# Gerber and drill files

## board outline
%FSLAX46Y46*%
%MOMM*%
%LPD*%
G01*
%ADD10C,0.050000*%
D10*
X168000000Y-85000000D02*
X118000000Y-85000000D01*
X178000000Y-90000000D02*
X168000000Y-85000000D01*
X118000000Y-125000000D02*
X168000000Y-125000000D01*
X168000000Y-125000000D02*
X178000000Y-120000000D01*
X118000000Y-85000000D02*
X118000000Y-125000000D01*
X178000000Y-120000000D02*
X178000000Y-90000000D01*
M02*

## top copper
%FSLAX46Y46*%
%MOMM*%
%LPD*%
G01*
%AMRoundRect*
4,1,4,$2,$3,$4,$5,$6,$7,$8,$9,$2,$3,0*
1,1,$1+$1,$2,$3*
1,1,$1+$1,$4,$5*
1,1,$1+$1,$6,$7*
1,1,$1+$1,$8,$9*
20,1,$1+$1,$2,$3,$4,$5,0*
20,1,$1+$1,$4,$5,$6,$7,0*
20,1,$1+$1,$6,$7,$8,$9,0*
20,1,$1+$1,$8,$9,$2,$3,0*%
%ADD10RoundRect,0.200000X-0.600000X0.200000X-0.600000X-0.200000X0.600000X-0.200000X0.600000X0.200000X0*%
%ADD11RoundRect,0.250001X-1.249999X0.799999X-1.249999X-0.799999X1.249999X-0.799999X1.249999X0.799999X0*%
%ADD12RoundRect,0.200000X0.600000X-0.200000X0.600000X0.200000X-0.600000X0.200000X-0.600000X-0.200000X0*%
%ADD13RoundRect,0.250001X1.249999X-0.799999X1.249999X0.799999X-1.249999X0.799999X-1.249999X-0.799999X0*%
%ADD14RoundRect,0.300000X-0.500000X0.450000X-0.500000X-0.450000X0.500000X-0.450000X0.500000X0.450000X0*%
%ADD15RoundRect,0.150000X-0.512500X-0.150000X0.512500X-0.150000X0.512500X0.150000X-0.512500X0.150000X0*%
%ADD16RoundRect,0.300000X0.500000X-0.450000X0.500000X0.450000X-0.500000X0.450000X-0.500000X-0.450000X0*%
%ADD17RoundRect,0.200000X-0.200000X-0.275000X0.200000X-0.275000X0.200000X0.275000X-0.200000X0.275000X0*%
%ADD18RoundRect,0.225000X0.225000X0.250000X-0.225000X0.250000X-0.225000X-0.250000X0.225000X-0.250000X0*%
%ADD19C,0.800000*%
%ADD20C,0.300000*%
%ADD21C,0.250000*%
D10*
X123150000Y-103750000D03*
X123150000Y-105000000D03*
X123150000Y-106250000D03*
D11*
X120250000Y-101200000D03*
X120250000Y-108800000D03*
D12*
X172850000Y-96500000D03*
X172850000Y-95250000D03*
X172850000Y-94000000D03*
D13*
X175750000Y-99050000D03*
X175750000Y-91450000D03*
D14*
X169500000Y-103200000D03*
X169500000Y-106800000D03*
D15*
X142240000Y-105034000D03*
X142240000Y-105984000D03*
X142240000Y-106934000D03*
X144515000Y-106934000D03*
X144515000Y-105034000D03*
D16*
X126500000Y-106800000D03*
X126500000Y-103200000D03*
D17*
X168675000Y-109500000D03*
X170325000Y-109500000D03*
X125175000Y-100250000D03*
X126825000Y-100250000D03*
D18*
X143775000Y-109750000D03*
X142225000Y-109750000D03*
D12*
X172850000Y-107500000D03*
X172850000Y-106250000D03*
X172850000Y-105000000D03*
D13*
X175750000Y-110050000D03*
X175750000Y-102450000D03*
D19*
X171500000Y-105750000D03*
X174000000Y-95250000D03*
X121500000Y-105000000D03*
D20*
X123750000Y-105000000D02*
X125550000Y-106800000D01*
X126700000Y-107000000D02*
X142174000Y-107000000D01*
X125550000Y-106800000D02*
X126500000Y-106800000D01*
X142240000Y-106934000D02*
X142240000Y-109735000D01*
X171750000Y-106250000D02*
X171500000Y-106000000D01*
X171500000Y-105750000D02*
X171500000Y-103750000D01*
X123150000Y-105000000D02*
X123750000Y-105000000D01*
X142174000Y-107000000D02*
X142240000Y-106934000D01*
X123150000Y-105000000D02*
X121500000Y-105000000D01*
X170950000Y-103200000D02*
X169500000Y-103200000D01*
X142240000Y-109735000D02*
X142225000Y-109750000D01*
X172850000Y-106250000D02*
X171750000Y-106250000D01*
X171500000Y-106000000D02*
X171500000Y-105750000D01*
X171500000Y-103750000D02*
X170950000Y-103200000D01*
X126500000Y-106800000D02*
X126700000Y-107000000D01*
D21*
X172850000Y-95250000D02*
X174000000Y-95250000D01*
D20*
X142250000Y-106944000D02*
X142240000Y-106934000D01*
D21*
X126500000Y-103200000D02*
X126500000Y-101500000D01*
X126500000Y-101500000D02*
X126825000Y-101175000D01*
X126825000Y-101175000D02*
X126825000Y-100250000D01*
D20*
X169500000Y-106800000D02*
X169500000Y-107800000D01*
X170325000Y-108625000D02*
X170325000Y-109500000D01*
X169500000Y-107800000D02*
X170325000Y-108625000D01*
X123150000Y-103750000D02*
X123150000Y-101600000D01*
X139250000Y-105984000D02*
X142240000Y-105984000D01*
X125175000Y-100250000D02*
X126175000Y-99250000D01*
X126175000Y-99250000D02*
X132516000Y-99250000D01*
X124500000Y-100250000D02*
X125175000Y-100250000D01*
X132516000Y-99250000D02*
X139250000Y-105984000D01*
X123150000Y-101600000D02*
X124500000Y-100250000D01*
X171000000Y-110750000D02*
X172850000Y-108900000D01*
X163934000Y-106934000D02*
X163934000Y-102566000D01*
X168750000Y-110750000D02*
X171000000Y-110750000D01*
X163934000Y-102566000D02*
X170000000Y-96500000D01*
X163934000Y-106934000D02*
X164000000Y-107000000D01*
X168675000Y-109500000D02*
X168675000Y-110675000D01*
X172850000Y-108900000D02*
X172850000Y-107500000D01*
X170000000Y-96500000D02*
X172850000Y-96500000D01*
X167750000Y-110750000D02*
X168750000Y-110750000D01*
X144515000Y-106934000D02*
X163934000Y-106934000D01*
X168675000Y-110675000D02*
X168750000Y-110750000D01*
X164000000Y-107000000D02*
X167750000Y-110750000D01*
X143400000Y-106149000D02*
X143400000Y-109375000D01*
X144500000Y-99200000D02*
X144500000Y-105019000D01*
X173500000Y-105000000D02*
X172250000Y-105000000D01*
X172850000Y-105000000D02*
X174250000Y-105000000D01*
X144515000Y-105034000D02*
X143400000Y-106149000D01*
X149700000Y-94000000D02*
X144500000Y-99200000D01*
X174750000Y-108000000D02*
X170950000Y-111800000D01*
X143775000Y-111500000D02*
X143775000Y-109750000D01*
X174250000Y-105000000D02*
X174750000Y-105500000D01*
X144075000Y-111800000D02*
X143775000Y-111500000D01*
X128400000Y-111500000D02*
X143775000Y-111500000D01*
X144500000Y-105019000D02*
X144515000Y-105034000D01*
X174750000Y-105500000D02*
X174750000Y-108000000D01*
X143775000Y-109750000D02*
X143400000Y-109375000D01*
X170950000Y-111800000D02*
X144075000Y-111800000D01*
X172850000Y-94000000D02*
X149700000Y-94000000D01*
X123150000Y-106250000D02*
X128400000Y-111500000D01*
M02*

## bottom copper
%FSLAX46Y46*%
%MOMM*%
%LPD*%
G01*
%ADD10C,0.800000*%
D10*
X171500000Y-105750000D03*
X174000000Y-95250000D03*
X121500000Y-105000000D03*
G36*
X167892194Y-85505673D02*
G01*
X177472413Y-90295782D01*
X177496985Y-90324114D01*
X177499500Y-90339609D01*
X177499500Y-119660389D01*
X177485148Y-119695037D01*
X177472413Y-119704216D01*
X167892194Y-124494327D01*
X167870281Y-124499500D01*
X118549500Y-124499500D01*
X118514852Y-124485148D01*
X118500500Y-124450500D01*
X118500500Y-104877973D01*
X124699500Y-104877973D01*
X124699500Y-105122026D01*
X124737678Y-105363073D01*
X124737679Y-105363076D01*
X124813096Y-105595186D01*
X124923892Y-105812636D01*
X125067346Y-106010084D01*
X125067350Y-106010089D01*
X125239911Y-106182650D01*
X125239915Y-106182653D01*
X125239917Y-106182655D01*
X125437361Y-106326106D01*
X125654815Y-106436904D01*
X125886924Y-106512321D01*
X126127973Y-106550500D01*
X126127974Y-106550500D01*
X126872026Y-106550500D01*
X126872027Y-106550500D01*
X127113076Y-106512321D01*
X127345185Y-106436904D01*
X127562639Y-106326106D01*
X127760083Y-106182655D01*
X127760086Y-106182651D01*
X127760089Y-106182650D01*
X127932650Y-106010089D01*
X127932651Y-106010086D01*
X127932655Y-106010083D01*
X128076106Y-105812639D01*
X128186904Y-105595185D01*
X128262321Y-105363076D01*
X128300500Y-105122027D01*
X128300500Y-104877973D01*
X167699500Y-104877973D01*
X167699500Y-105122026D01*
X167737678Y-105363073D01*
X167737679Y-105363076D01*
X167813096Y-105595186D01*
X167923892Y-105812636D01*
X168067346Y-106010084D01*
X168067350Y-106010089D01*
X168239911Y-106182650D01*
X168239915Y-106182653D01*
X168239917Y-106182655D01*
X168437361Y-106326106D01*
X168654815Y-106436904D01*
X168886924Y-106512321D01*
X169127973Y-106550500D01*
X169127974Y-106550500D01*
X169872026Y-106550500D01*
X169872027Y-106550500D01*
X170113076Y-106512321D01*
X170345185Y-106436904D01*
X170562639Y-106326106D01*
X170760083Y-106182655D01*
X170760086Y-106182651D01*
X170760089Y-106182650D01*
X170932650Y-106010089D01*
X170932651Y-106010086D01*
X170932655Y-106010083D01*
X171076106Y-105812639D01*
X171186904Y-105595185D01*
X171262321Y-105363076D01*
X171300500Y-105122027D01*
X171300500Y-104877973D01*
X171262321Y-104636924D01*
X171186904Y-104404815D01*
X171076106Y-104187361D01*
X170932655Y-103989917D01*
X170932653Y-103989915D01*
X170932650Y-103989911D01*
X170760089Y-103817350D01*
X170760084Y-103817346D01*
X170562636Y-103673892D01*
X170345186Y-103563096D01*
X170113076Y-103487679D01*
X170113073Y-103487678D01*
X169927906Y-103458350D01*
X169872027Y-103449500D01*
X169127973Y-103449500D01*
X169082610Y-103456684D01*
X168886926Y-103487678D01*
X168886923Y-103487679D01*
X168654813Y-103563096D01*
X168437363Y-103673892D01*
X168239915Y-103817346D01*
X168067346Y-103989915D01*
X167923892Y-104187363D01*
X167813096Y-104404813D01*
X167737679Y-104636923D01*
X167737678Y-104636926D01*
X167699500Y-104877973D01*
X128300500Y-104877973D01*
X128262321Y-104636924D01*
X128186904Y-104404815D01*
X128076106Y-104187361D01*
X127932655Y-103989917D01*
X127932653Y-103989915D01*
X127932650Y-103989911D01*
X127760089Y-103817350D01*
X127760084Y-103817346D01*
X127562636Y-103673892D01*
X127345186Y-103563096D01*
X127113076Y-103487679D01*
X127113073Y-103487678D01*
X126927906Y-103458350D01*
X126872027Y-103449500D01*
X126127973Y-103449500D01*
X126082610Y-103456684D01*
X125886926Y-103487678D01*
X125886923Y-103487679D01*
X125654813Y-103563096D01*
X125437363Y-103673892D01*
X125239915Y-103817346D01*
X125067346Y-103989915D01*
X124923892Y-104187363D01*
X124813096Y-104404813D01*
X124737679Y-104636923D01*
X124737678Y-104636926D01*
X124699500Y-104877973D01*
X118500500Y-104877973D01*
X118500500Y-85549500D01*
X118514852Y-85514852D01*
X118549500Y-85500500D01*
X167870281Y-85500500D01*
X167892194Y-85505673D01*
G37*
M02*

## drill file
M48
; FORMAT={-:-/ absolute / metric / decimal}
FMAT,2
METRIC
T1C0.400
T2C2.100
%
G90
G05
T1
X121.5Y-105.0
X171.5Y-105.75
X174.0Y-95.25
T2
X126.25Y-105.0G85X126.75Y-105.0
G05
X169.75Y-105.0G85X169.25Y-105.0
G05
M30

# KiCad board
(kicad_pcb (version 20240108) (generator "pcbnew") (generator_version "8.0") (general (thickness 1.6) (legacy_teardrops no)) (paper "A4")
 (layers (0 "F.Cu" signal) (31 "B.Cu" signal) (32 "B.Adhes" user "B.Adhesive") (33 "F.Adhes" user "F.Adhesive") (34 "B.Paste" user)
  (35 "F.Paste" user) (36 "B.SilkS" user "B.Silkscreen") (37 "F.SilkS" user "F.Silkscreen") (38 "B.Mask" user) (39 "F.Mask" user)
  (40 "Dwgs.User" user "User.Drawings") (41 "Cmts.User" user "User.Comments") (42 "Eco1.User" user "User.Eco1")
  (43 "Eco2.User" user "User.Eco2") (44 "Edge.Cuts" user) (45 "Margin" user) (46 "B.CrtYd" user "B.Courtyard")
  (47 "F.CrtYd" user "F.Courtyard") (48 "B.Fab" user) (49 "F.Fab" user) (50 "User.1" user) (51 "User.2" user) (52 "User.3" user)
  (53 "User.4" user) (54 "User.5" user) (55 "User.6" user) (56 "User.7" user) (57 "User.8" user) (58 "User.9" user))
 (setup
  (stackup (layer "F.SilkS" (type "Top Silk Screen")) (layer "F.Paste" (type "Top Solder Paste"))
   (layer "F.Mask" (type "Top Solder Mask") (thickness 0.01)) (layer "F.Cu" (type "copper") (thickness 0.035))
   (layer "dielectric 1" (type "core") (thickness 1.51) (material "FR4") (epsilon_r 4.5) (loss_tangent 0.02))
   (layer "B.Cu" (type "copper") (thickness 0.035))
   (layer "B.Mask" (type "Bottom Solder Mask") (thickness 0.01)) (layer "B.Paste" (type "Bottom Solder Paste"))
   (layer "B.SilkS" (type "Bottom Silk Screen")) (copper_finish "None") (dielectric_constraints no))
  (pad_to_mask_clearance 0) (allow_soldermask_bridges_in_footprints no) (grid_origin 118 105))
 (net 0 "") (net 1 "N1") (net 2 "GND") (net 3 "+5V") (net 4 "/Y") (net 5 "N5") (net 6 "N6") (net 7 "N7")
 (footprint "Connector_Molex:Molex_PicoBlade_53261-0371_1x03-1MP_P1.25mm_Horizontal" (layer "F.Cu") (at 120.75 105 -90)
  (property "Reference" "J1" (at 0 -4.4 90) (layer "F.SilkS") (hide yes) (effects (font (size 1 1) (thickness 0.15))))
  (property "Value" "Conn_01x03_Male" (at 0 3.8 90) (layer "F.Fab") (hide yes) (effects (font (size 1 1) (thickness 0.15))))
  (pad "1" smd roundrect (at -1.25 -2.4 270) (size 0.8 1.6) (layers "F.Cu" "F.Paste" "F.Mask") (roundrect_rratio 0.25) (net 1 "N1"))
  (pad "2" smd roundrect (at 0 -2.4 270) (size 0.8 1.6) (layers "F.Cu" "F.Paste" "F.Mask") (roundrect_rratio 0.25) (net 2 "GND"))
  (pad "3" smd roundrect (at 1.25 -2.4 270) (size 0.8 1.6) (layers "F.Cu" "F.Paste" "F.Mask") (roundrect_rratio 0.25) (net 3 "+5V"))
  (pad "MP" smd roundrect (at -3.8 0.5 270) (size 2.1 3) (layers "F.Cu" "F.Paste" "F.Mask") (roundrect_rratio 0.1190480952))
  (pad "MP" smd roundrect (at 3.8 0.5 270) (size 2.1 3) (layers "F.Cu" "F.Paste" "F.Mask") (roundrect_rratio 0.1190480952)))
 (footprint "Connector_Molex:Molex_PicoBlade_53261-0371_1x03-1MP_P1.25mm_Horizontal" (layer "F.Cu") (at 175.25 95.25 90)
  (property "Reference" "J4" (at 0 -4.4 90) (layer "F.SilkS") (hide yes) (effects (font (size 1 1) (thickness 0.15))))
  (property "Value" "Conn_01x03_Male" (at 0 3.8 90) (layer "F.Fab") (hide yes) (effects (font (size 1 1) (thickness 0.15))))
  (pad "1" smd roundrect (at -1.25 -2.4 90) (size 0.8 1.6) (layers "F.Cu" "F.Paste" "F.Mask") (roundrect_rratio 0.25) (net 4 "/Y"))
  (pad "2" smd roundrect (at 0 -2.4 90) (size 0.8 1.6) (layers "F.Cu" "F.Paste" "F.Mask") (roundrect_rratio 0.25) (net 2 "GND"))
  (pad "3" smd roundrect (at 1.25 -2.4 90) (size 0.8 1.6) (layers "F.Cu" "F.Paste" "F.Mask") (roundrect_rratio 0.25) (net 3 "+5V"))
  (pad "MP" smd roundrect (at -3.8 0.5 90) (size 2.1 3) (layers "F.Cu" "F.Paste" "F.Mask") (roundrect_rratio 0.1190480952))
  (pad "MP" smd roundrect (at 3.8 0.5 90) (size 2.1 3) (layers "F.Cu" "F.Paste" "F.Mask") (roundrect_rratio 0.1190480952)))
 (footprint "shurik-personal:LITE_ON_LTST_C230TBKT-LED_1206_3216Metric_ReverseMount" (layer "F.Cu") (at 169.5 105 -90)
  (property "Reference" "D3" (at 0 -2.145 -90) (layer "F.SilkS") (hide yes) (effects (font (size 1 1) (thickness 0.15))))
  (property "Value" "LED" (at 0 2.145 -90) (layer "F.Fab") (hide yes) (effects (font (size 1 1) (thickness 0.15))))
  (pad "" np_thru_hole oval (at 0 0 270) (size 2.1 2.6) (drill oval 2.1 2.6) (layers "F&B.Cu" "*.Mask"))
  (pad "1" smd roundrect (at -1.8 0 270) (size 1.5 1.6) (layers "F.Cu" "F.Paste" "F.Mask") (roundrect_rratio 0.2) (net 2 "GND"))
  (pad "2" smd roundrect (at 1.8 0 270) (size 1.5 1.6) (layers "F.Cu" "F.Paste" "F.Mask") (roundrect_rratio 0.2) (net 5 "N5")))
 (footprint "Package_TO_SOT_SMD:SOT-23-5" (layer "F.Cu") (at 143.3775 105.984)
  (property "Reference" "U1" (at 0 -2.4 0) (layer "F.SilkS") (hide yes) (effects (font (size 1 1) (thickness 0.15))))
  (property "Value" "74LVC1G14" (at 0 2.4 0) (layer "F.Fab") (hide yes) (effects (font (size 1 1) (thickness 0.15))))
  (pad "1" smd roundrect (at -1.1375 -0.95) (size 1.325 0.6) (layers "F.Cu" "F.Paste" "F.Mask") (roundrect_rratio 0.25) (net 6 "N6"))
  (pad "2" smd roundrect (at -1.1375 0) (size 1.325 0.6) (layers "F.Cu" "F.Paste" "F.Mask") (roundrect_rratio 0.25) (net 1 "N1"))
  (pad "3" smd roundrect (at -1.1375 0.95) (size 1.325 0.6) (layers "F.Cu" "F.Paste" "F.Mask") (roundrect_rratio 0.25) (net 2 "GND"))
  (pad "4" smd roundrect (at 1.1375 0.95) (size 1.325 0.6) (layers "F.Cu" "F.Paste" "F.Mask") (roundrect_rratio 0.25) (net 4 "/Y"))
  (pad "5" smd roundrect (at 1.1375 -0.95) (size 1.325 0.6) (layers "F.Cu" "F.Paste" "F.Mask") (roundrect_rratio 0.25) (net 3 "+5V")))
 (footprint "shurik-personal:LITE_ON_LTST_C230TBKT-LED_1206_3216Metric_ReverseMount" (layer "F.Cu") (at 126.5 105 90)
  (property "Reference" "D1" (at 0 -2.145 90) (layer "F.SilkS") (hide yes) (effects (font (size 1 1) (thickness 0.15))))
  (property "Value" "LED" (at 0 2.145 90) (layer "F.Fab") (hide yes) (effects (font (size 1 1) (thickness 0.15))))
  (pad "" np_thru_hole oval (at 0 0 90) (size 2.1 2.6) (drill oval 2.1 2.6) (layers "F&B.Cu" "*.Mask"))
  (pad "1" smd roundrect (at -1.8 0 90) (size 1.5 1.6) (layers "F.Cu" "F.Paste" "F.Mask") (roundrect_rratio 0.2) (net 2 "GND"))
  (pad "2" smd roundrect (at 1.8 0 90) (size 1.5 1.6) (layers "F.Cu" "F.Paste" "F.Mask") (roundrect_rratio 0.2) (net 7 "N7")))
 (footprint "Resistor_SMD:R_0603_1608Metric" (layer "F.Cu") (at 169.5 109.5)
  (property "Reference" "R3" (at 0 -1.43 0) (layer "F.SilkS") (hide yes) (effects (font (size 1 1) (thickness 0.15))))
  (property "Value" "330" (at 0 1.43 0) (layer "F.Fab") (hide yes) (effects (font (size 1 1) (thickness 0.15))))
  (pad "1" smd roundrect (at -0.825 0) (size 0.8 0.95) (layers "F.Cu" "F.Paste" "F.Mask") (roundrect_rratio 0.25) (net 4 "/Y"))
  (pad "2" smd roundrect (at 0.825 0) (size 0.8 0.95) (layers "F.Cu" "F.Paste" "F.Mask") (roundrect_rratio 0.25) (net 5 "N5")))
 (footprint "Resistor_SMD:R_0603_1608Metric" (layer "F.Cu") (at 126 100.25)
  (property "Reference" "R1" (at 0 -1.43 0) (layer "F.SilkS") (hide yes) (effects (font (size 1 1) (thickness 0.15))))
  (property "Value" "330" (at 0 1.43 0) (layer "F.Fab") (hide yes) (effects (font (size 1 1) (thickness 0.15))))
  (pad "1" smd roundrect (at -0.825 0) (size 0.8 0.95) (layers "F.Cu" "F.Paste" "F.Mask") (roundrect_rratio 0.25) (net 1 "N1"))
  (pad "2" smd roundrect (at 0.825 0) (size 0.8 0.95) (layers "F.Cu" "F.Paste" "F.Mask") (roundrect_rratio 0.25) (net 7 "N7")))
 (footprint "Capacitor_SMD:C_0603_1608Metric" (layer "F.Cu") (at 143 109.75 180)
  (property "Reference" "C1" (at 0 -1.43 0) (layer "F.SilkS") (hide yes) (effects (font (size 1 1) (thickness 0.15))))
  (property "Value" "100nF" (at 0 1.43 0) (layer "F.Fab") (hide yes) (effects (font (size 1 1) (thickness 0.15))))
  (pad "1" smd roundrect (at -0.775 0 180) (size 0.9 0.95) (layers "F.Cu" "F.Paste" "F.Mask") (roundrect_rratio 0.25) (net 3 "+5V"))
  (pad "2" smd roundrect (at 0.775 0 180) (size 0.9 0.95) (layers "F.Cu" "F.Paste" "F.Mask") (roundrect_rratio 0.25) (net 2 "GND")))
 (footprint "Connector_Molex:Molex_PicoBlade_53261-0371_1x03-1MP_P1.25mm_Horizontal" (layer "F.Cu") (at 175.25 106.25 90)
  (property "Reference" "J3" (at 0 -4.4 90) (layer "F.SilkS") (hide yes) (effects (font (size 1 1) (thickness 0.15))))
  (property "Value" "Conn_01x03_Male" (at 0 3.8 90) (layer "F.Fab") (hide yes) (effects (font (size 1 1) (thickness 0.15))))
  (pad "1" smd roundrect (at -1.25 -2.4 90) (size 0.8 1.6) (layers "F.Cu" "F.Paste" "F.Mask") (roundrect_rratio 0.25) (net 4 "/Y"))
  (pad "2" smd roundrect (at 0 -2.4 90) (size 0.8 1.6) (layers "F.Cu" "F.Paste" "F.Mask") (roundrect_rratio 0.25) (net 2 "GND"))
  (pad "3" smd roundrect (at 1.25 -2.4 90) (size 0.8 1.6) (layers "F.Cu" "F.Paste" "F.Mask") (roundrect_rratio 0.25) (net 3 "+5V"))
  (pad "MP" smd roundrect (at -3.8 0.5 90) (size 2.1 3) (layers "F.Cu" "F.Paste" "F.Mask") (roundrect_rratio 0.1190480952))
  (pad "MP" smd roundrect (at 3.8 0.5 90) (size 2.1 3) (layers "F.Cu" "F.Paste" "F.Mask") (roundrect_rratio 0.1190480952)))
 (gr_line (start 168 85) (end 118 85) (stroke (width 0.05) (type solid)) (layer "Edge.Cuts"))
 (gr_line (start 178 90) (end 168 85) (stroke (width 0.05) (type solid)) (layer "Edge.Cuts"))
 (gr_line (start 118 125) (end 168 125) (stroke (width 0.05) (type solid)) (layer "Edge.Cuts"))
 (gr_line (start 168 125) (end 178 120) (stroke (width 0.05) (type solid)) (layer "Edge.Cuts"))
 (gr_line (start 118 85) (end 118 125) (stroke (width 0.05) (type solid)) (layer "Edge.Cuts"))
 (gr_line (start 178 120) (end 178 90) (stroke (width 0.05) (type solid)) (layer "Edge.Cuts"))
 (segment (start 123.75 105) (end 125.55 106.8) (width 0.3) (layer "F.Cu") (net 2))
 (segment (start 126.7 107) (end 142.174 107) (width 0.3) (layer "F.Cu") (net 2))
 (segment (start 125.55 106.8) (end 126.5 106.8) (width 0.3) (layer "F.Cu") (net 2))
 (segment (start 142.24 106.934) (end 142.24 109.735) (width 0.3) (layer "F.Cu") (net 2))
 (segment (start 171.75 106.25) (end 171.5 106) (width 0.3) (layer "F.Cu") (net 2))
 (segment (start 171.5 105.75) (end 171.5 103.75) (width 0.3) (layer "F.Cu") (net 2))
 (segment (start 123.15 105) (end 123.75 105) (width 0.3) (layer "F.Cu") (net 2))
 (segment (start 142.174 107) (end 142.24 106.934) (width 0.3) (layer "F.Cu") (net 2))
 (segment (start 123.15 105) (end 121.5 105) (width 0.3) (layer "F.Cu") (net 2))
 (segment (start 170.95 103.2) (end 169.5 103.2) (width 0.3) (layer "F.Cu") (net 2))
 (segment (start 142.24 109.735) (end 142.225 109.75) (width 0.3) (layer "F.Cu") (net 2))
 (segment (start 172.85 106.25) (end 171.75 106.25) (width 0.3) (layer "F.Cu") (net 2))
 (segment (start 171.5 106) (end 171.5 105.75) (width 0.3) (layer "F.Cu") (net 2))
 (segment (start 171.5 103.75) (end 170.95 103.2) (width 0.3) (layer "F.Cu") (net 2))
 (segment (start 126.5 106.8) (end 126.7 107) (width 0.3) (layer "F.Cu") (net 2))
 (segment (start 172.85 95.25) (end 174 95.25) (width 0.25) (layer "F.Cu") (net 2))
 (segment (start 142.25 106.944) (end 142.24 106.934) (width 0.3) (layer "F.Cu") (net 2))
 (via (at 171.5 105.75) (size 0.8) (drill 0.4) (layers "F.Cu" "B.Cu") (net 2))
 (via (at 174 95.25) (size 0.8) (drill 0.4) (layers "F.Cu" "B.Cu") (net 2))
 (via (at 121.5 105) (size 0.8) (drill 0.4) (layers "F.Cu" "B.Cu") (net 2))
 (segment (start 126.5 103.2) (end 126.5 101.5) (width 0.25) (layer "F.Cu") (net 7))
 (segment (start 126.5 101.5) (end 126.825 101.175) (width 0.25) (layer "F.Cu") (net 7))
 (segment (start 126.825 101.175) (end 126.825 100.25) (width 0.25) (layer "F.Cu") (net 7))
 (segment (start 169.5 106.8) (end 169.5 107.8) (width 0.3) (layer "F.Cu") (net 5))
 (segment (start 170.325 108.625) (end 170.325 109.5) (width 0.3) (layer "F.Cu") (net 5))
 (segment (start 169.5 107.8) (end 170.325 108.625) (width 0.3) (layer "F.Cu") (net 5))
 (segment (start 123.15 103.75) (end 123.15 101.6) (width 0.3) (layer "F.Cu") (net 1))
 (segment (start 139.25 105.984) (end 142.24 105.984) (width 0.3) (layer "F.Cu") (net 1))
 (segment (start 125.175 100.25) (end 126.175 99.25) (width 0.3) (layer "F.Cu") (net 1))
 (segment (start 126.175 99.25) (end 132.516 99.25) (width 0.3) (layer "F.Cu") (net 1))
 (segment (start 124.5 100.25) (end 125.175 100.25) (width 0.3) (layer "F.Cu") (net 1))
 (segment (start 132.516 99.25) (end 139.25 105.984) (width 0.3) (layer "F.Cu") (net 1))
 (segment (start 123.15 101.6) (end 124.5 100.25) (width 0.3) (layer "F.Cu") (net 1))
 (segment (start 171 110.75) (end 172.85 108.9) (width 0.3) (layer "F.Cu") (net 4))
 (segment (start 163.934 106.934) (end 163.934 102.566) (width 0.3) (layer "F.Cu") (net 4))
 (segment (start 168.75 110.75) (end 171 110.75) (width 0.3) (layer "F.Cu") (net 4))
 (segment (start 163.934 102.566) (end 170 96.5) (width 0.3) (layer "F.Cu") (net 4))
 (segment (start 163.934 106.934) (end 164 107) (width 0.3) (layer "F.Cu") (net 4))
 (segment (start 168.675 109.5) (end 168.675 110.675) (width 0.3) (layer "F.Cu") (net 4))
 (segment (start 172.85 108.9) (end 172.85 107.5) (width 0.3) (layer "F.Cu") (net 4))
 (segment (start 170 96.5) (end 172.85 96.5) (width 0.3) (layer "F.Cu") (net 4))
 (segment (start 167.75 110.75) (end 168.75 110.75) (width 0.3) (layer "F.Cu") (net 4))
 (segment (start 144.515 106.934) (end 163.934 106.934) (width 0.3) (layer "F.Cu") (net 4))
 (segment (start 168.675 110.675) (end 168.75 110.75) (width 0.3) (layer "F.Cu") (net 4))
 (segment (start 164 107) (end 167.75 110.75) (width 0.3) (layer "F.Cu") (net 4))
 (segment (start 143.4 106.149) (end 143.4 109.375) (width 0.3) (layer "F.Cu") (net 3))
 (segment (start 144.5 99.2) (end 144.5 105.019) (width 0.3) (layer "F.Cu") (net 3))
 (segment (start 173.5 105) (end 172.25 105) (width 0.3) (layer "F.Cu") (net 3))
 (segment (start 172.85 105) (end 174.25 105) (width 0.3) (layer "F.Cu") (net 3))
 (segment (start 144.515 105.034) (end 143.4 106.149) (width 0.3) (layer "F.Cu") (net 3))
 (segment (start 149.7 94) (end 144.5 99.2) (width 0.3) (layer "F.Cu") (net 3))
 (segment (start 174.75 108) (end 170.95 111.8) (width 0.3) (layer "F.Cu") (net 3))
 (segment (start 143.775 111.5) (end 143.775 109.75) (width 0.3) (layer "F.Cu") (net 3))
 (segment (start 174.25 105) (end 174.75 105.5) (width 0.3) (layer "F.Cu") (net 3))
 (segment (start 144.075 111.8) (end 143.775 111.5) (width 0.3) (layer "F.Cu") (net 3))
 (segment (start 128.4 111.5) (end 143.775 111.5) (width 0.3) (layer "F.Cu") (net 3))
 (segment (start 144.5 105.019) (end 144.515 105.034) (width 0.3) (layer "F.Cu") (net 3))
 (segment (start 174.75 105.5) (end 174.75 108) (width 0.3) (layer "F.Cu") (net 3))
 (segment (start 143.775 109.75) (end 143.4 109.375) (width 0.3) (layer "F.Cu") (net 3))
 (segment (start 170.95 111.8) (end 144.075 111.8) (width 0.3) (layer "F.Cu") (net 3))
 (segment (start 172.85 94) (end 149.7 94) (width 0.3) (layer "F.Cu") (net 3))
 (segment (start 123.15 106.25) (end 128.4 111.5) (width 0.3) (layer "F.Cu") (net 3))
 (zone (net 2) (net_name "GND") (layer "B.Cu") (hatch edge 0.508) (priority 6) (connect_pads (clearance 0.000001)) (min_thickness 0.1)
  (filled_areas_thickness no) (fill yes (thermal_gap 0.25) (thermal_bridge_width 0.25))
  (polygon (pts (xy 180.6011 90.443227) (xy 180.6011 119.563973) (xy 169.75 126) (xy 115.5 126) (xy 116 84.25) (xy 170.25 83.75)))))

